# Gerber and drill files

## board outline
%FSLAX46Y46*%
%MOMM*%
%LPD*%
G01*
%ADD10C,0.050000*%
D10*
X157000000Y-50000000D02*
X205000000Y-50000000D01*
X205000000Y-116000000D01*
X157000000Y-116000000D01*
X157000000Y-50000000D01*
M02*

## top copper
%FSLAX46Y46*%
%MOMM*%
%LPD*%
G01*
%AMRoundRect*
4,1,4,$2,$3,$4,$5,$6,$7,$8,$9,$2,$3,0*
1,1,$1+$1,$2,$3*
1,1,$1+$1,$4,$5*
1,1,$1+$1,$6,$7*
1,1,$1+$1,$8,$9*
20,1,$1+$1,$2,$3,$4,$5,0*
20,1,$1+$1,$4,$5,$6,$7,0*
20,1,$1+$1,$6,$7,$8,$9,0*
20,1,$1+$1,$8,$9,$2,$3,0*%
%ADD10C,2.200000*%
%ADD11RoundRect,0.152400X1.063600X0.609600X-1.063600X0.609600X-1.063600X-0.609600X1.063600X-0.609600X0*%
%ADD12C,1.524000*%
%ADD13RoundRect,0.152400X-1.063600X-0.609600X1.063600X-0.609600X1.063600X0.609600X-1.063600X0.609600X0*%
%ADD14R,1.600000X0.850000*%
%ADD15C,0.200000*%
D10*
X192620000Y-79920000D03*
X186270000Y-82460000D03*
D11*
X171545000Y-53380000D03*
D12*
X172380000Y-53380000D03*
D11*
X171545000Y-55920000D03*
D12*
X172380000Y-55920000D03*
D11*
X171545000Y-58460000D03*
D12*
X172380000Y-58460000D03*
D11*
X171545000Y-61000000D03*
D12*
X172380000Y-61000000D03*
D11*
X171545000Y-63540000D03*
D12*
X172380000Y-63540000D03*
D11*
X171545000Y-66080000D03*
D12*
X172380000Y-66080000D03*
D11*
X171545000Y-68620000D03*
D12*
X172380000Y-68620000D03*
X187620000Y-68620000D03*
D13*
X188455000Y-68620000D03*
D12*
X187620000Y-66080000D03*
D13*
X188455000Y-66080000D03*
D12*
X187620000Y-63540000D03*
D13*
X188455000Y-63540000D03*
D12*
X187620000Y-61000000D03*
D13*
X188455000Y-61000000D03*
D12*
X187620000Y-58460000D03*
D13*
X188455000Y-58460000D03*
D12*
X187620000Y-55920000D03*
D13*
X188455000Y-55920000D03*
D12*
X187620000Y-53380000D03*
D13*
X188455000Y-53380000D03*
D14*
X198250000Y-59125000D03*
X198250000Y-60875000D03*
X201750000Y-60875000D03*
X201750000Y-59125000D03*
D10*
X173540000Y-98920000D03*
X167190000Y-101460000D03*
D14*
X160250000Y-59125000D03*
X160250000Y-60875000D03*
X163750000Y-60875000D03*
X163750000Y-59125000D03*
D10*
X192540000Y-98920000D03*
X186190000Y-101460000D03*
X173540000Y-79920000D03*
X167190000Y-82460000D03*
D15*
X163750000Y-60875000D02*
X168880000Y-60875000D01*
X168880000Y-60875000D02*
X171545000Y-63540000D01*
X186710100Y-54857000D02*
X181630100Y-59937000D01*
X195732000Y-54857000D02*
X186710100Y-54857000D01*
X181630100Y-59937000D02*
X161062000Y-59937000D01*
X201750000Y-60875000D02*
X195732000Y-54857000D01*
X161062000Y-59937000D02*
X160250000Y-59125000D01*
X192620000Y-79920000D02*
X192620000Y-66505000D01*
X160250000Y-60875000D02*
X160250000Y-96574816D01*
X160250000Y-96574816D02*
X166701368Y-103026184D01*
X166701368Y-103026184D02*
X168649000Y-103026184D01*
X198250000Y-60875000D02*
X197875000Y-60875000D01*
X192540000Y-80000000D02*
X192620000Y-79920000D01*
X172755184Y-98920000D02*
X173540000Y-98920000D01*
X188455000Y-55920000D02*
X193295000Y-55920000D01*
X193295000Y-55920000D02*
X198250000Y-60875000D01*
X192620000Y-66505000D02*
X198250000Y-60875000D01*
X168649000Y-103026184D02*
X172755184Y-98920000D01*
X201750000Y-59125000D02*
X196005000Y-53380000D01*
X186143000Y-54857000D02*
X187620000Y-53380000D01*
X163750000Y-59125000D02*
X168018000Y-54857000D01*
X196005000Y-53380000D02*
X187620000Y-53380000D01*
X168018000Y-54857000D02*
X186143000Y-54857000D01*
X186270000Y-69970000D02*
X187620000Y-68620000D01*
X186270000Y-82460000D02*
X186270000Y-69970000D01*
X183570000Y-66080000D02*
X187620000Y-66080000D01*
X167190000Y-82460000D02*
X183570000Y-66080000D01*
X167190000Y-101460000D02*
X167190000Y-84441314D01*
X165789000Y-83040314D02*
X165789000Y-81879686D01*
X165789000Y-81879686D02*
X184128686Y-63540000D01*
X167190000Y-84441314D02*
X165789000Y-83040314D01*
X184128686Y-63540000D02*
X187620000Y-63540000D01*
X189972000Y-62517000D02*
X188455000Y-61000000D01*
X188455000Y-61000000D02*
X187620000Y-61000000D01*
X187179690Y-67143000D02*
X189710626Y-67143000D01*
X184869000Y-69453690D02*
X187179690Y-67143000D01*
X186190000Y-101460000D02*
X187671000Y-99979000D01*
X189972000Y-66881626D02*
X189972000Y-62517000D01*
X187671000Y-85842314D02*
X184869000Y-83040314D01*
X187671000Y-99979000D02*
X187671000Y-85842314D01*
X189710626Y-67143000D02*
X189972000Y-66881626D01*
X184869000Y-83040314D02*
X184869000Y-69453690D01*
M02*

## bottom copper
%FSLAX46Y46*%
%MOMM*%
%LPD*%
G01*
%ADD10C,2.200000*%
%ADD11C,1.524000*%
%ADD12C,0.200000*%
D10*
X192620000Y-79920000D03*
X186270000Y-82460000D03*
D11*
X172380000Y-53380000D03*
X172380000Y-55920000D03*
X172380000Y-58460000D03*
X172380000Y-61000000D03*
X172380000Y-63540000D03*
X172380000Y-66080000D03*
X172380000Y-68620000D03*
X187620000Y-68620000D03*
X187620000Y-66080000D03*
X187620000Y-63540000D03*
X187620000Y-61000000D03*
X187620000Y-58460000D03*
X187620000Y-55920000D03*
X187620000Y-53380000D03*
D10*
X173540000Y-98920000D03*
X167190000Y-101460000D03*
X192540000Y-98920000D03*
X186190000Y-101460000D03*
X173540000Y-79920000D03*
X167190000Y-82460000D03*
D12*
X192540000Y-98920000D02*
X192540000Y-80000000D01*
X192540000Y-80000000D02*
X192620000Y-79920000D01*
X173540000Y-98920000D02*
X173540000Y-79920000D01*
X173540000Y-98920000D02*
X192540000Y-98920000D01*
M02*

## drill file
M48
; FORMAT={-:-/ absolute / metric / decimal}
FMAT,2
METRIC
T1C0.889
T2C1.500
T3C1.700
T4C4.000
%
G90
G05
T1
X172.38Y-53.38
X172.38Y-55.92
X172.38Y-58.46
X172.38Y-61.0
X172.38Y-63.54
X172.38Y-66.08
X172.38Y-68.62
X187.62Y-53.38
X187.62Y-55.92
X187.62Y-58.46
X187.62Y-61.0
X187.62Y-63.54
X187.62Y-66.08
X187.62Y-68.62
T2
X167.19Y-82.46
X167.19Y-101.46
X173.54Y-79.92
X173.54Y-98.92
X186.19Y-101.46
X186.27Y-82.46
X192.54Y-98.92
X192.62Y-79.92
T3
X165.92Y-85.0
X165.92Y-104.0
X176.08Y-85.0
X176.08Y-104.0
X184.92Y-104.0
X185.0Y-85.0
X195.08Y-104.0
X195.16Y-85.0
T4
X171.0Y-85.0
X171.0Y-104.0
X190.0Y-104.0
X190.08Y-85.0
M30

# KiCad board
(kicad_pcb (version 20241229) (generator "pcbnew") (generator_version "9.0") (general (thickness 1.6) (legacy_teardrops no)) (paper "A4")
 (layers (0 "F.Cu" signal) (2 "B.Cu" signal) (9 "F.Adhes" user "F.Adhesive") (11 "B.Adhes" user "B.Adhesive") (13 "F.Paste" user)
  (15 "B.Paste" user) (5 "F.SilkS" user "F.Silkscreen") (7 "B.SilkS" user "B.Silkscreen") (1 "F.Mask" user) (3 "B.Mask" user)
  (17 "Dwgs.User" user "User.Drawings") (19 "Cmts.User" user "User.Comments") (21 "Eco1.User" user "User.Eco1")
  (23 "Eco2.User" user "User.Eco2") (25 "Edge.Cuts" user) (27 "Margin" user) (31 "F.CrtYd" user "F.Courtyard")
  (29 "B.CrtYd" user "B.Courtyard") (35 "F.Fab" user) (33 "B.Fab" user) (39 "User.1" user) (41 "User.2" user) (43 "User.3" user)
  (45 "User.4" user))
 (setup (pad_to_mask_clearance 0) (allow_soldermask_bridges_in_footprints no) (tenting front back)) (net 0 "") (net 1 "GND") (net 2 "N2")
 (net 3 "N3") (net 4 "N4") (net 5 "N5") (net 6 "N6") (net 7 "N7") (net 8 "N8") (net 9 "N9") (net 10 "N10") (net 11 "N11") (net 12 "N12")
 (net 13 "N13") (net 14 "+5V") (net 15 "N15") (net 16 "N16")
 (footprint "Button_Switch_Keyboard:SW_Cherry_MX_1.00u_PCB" (layer "F.Cu") (at 192.62 79.92)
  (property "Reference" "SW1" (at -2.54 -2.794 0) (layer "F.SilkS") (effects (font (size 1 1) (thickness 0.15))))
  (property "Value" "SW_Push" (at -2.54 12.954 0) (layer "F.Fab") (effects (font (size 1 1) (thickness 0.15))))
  (pad "" np_thru_hole circle (at -7.62 5.08) (size 1.7 1.7) (drill 1.7) (layers "*.Cu" "*.Mask"))
  (pad "" np_thru_hole circle (at -2.54 5.08) (size 4 4) (drill 4) (layers "*.Cu" "*.Mask"))
  (pad "" np_thru_hole circle (at 2.54 5.08) (size 1.7 1.7) (drill 1.7) (layers "*.Cu" "*.Mask"))
  (pad "1" thru_hole circle (at 0 0) (size 2.2 2.2) (drill 1.5) (layers "*.Cu" "*.Mask") (remove_unused_layers no) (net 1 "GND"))
  (pad "2" thru_hole circle (at -6.35 2.54) (size 2.2 2.2) (drill 1.5) (layers "*.Cu" "*.Mask") (remove_unused_layers no) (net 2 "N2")))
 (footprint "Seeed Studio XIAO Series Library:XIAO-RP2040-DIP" (layer "F.Cu") (at 180 61)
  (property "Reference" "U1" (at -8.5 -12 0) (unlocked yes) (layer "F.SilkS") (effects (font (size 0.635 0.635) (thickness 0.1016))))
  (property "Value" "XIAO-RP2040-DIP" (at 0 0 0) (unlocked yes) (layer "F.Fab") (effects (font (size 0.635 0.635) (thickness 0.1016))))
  (pad "1" smd roundrect (at -8.455 -7.62 180) (size 2.432 1.524) (layers "F.Cu" "F.Mask") (roundrect_rratio 0.1) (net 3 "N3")
   (thermal_bridge_angle 45))
  (pad "1" thru_hole circle (at -7.62 -7.62 180) (size 1.524 1.524) (drill 0.889) (layers "*.Cu" "*.Mask") (remove_unused_layers no)
   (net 3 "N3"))
  (pad "2" smd roundrect (at -8.455 -5.08 180) (size 2.432 1.524) (layers "F.Cu" "F.Mask") (roundrect_rratio 0.1) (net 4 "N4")
   (thermal_bridge_angle 45))
  (pad "2" thru_hole circle (at -7.62 -5.08 180) (size 1.524 1.524) (drill 0.889) (layers "*.Cu" "*.Mask") (remove_unused_layers no)
   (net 4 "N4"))
  (pad "3" smd roundrect (at -8.455 -2.54 180) (size 2.432 1.524) (layers "F.Cu" "F.Mask") (roundrect_rratio 0.1) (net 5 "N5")
   (thermal_bridge_angle 45))
  (pad "3" thru_hole circle (at -7.62 -2.54 180) (size 1.524 1.524) (drill 0.889) (layers "*.Cu" "*.Mask") (remove_unused_layers no)
   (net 5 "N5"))
  (pad "4" smd roundrect (at -8.455 0 180) (size 2.432 1.524) (layers "F.Cu" "F.Mask") (roundrect_rratio 0.1) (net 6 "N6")
   (thermal_bridge_angle 45))
  (pad "4" thru_hole circle (at -7.62 0 180) (size 1.524 1.524) (drill 0.889) (layers "*.Cu" "*.Mask") (remove_unused_layers no)
   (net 6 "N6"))
  (pad "5" smd roundrect (at -8.455 2.54 180) (size 2.432 1.524) (layers "F.Cu" "F.Mask") (roundrect_rratio 0.1) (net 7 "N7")
   (thermal_bridge_angle 45))
  (pad "5" thru_hole circle (at -7.62 2.54 180) (size 1.524 1.524) (drill 0.889) (layers "*.Cu" "*.Mask") (remove_unused_layers no)
   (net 7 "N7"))
  (pad "6" smd roundrect (at -8.455 5.08 180) (size 2.432 1.524) (layers "F.Cu" "F.Mask") (roundrect_rratio 0.1) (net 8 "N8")
   (thermal_bridge_angle 45))
  (pad "6" thru_hole circle (at -7.62 5.08 180) (size 1.524 1.524) (drill 0.889) (layers "*.Cu" "*.Mask") (remove_unused_layers no)
   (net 8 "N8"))
  (pad "7" smd roundrect (at -8.455 7.62 180) (size 2.432 1.524) (layers "F.Cu" "F.Mask") (roundrect_rratio 0.1) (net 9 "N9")
   (thermal_bridge_angle 45))
  (pad "7" thru_hole circle (at -7.62 7.62 180) (size 1.524 1.524) (drill 0.889) (layers "*.Cu" "*.Mask") (remove_unused_layers no)
   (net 9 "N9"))
  (pad "8" thru_hole circle (at 7.62 7.62) (size 1.524 1.524) (drill 0.889) (layers "*.Cu" "*.Mask") (remove_unused_layers no) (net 2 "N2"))
  (pad "8" smd roundrect (at 8.455 7.62) (size 2.432 1.524) (layers "F.Cu" "F.Mask") (roundrect_rratio 0.1) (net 2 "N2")
   (thermal_bridge_angle 45))
  (pad "9" thru_hole circle (at 7.62 5.08) (size 1.524 1.524) (drill 0.889) (layers "*.Cu" "*.Mask") (remove_unused_layers no)
   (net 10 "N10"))
  (pad "9" smd roundrect (at 8.455 5.08) (size 2.432 1.524) (layers "F.Cu" "F.Mask") (roundrect_rratio 0.1) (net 10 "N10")
   (thermal_bridge_angle 45))
  (pad "10" thru_hole circle (at 7.62 2.54) (size 1.524 1.524) (drill 0.889) (layers "*.Cu" "*.Mask") (remove_unused_layers no)
   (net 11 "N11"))
  (pad "10" smd roundrect (at 8.455 2.54) (size 2.432 1.524) (layers "F.Cu" "F.Mask") (roundrect_rratio 0.1) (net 11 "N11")
   (thermal_bridge_angle 45))
  (pad "11" thru_hole circle (at 7.62 0) (size 1.524 1.524) (drill 0.889) (layers "*.Cu" "*.Mask") (remove_unused_layers no) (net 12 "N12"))
  (pad "11" smd roundrect (at 8.455 0) (size 2.432 1.524) (layers "F.Cu" "F.Mask") (roundrect_rratio 0.1) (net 12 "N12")
   (thermal_bridge_angle 45))
  (pad "12" thru_hole circle (at 7.62 -2.54) (size 1.524 1.524) (drill 0.889) (layers "*.Cu" "*.Mask") (remove_unused_layers no)
   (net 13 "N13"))
  (pad "12" smd roundrect (at 8.455 -2.54) (size 2.432 1.524) (layers "F.Cu" "F.Mask") (roundrect_rratio 0.1) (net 13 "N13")
   (thermal_bridge_angle 45))
  (pad "13" thru_hole circle (at 7.62 -5.08) (size 1.524 1.524) (drill 0.889) (layers "*.Cu" "*.Mask") (remove_unused_layers no)
   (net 1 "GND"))
  (pad "13" smd roundrect (at 8.455 -5.08) (size 2.432 1.524) (layers "F.Cu" "F.Mask") (roundrect_rratio 0.1) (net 1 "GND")
   (thermal_bridge_angle 45))
  (pad "14" thru_hole circle (at 7.62 -7.62) (size 1.524 1.524) (drill 0.889) (layers "*.Cu" "*.Mask") (remove_unused_layers no)
   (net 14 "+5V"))
  (pad "14" smd roundrect (at 8.455 -7.62) (size 2.432 1.524) (layers "F.Cu" "F.Mask") (roundrect_rratio 0.1) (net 14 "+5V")
   (thermal_bridge_angle 45)))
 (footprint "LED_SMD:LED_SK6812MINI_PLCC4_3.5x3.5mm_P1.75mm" (layer "F.Cu") (at 200 60)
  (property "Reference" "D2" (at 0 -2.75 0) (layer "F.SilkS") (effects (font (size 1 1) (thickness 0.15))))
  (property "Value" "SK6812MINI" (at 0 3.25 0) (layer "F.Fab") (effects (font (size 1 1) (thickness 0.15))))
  (pad "1" smd rect (at -1.75 -0.875) (size 1.6 0.85) (layers "F.Cu" "F.Mask" "F.Paste") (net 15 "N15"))
  (pad "2" smd rect (at -1.75 0.875) (size 1.6 0.85) (layers "F.Cu" "F.Mask" "F.Paste") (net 1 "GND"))
  (pad "3" smd rect (at 1.75 0.875) (size 1.6 0.85) (layers "F.Cu" "F.Mask" "F.Paste") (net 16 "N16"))
  (pad "4" smd rect (at 1.75 -0.875) (size 1.6 0.85) (layers "F.Cu" "F.Mask" "F.Paste") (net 14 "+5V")))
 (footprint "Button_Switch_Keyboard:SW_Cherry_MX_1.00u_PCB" (layer "F.Cu") (at 173.54 98.92)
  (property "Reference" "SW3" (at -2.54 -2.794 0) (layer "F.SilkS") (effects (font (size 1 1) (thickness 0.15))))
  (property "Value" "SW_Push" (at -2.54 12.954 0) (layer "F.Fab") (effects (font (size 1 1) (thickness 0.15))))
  (pad "" np_thru_hole circle (at -7.62 5.08) (size 1.7 1.7) (drill 1.7) (layers "*.Cu" "*.Mask"))
  (pad "" np_thru_hole circle (at -2.54 5.08) (size 4 4) (drill 4) (layers "*.Cu" "*.Mask"))
  (pad "" np_thru_hole circle (at 2.54 5.08) (size 1.7 1.7) (drill 1.7) (layers "*.Cu" "*.Mask"))
  (pad "1" thru_hole circle (at 0 0) (size 2.2 2.2) (drill 1.5) (layers "*.Cu" "*.Mask") (remove_unused_layers no) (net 1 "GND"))
  (pad "2" thru_hole circle (at -6.35 2.54) (size 2.2 2.2) (drill 1.5) (layers "*.Cu" "*.Mask") (remove_unused_layers no) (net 11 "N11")))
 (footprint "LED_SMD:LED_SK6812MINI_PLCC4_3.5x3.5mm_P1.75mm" (layer "F.Cu") (at 162 60)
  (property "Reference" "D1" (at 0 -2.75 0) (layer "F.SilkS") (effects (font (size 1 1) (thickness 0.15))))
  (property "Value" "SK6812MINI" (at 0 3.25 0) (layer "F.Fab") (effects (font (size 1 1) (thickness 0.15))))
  (pad "1" smd rect (at -1.75 -0.875) (size 1.6 0.85) (layers "F.Cu" "F.Mask" "F.Paste") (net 16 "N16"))
  (pad "2" smd rect (at -1.75 0.875) (size 1.6 0.85) (layers "F.Cu" "F.Mask" "F.Paste") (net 1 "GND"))
  (pad "3" smd rect (at 1.75 0.875) (size 1.6 0.85) (layers "F.Cu" "F.Mask" "F.Paste") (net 7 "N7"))
  (pad "4" smd rect (at 1.75 -0.875) (size 1.6 0.85) (layers "F.Cu" "F.Mask" "F.Paste") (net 14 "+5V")))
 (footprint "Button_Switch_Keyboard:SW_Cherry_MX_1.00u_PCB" (layer "F.Cu") (at 192.54 98.92)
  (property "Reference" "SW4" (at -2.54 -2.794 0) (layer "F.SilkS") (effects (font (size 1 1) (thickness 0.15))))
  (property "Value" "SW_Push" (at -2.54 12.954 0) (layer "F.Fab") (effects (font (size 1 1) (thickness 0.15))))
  (pad "" np_thru_hole circle (at -7.62 5.08) (size 1.7 1.7) (drill 1.7) (layers "*.Cu" "*.Mask"))
  (pad "" np_thru_hole circle (at -2.54 5.08) (size 4 4) (drill 4) (layers "*.Cu" "*.Mask"))
  (pad "" np_thru_hole circle (at 2.54 5.08) (size 1.7 1.7) (drill 1.7) (layers "*.Cu" "*.Mask"))
  (pad "1" thru_hole circle (at 0 0) (size 2.2 2.2) (drill 1.5) (layers "*.Cu" "*.Mask") (remove_unused_layers no) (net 1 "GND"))
  (pad "2" thru_hole circle (at -6.35 2.54) (size 2.2 2.2) (drill 1.5) (layers "*.Cu" "*.Mask") (remove_unused_layers no) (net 12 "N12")))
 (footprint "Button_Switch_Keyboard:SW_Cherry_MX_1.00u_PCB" (layer "F.Cu") (at 173.54 79.92)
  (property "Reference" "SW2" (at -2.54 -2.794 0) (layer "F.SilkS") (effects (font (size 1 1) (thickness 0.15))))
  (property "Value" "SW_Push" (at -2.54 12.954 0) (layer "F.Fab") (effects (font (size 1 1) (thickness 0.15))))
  (pad "" np_thru_hole circle (at -7.62 5.08) (size 1.7 1.7) (drill 1.7) (layers "*.Cu" "*.Mask"))
  (pad "" np_thru_hole circle (at -2.54 5.08) (size 4 4) (drill 4) (layers "*.Cu" "*.Mask"))
  (pad "" np_thru_hole circle (at 2.54 5.08) (size 1.7 1.7) (drill 1.7) (layers "*.Cu" "*.Mask"))
  (pad "1" thru_hole circle (at 0 0) (size 2.2 2.2) (drill 1.5) (layers "*.Cu" "*.Mask") (remove_unused_layers no) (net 1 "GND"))
  (pad "2" thru_hole circle (at -6.35 2.54) (size 2.2 2.2) (drill 1.5) (layers "*.Cu" "*.Mask") (remove_unused_layers no) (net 10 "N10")))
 (gr_rect (start 157 50) (end 205 116) (stroke (width 0.05) (type default)) (fill no) (layer "Edge.Cuts"))
 (segment (start 163.75 60.875) (end 168.88 60.875) (width 0.2) (layer "F.Cu") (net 7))
 (segment (start 168.88 60.875) (end 171.545 63.54) (width 0.2) (layer "F.Cu") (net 7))
 (segment (start 186.7101 54.857) (end 181.6301 59.937) (width 0.2) (layer "F.Cu") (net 16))
 (segment (start 195.732 54.857) (end 186.7101 54.857) (width 0.2) (layer "F.Cu") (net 16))
 (segment (start 181.6301 59.937) (end 161.062 59.937) (width 0.2) (layer "F.Cu") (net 16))
 (segment (start 201.75 60.875) (end 195.732 54.857) (width 0.2) (layer "F.Cu") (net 16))
 (segment (start 161.062 59.937) (end 160.25 59.125) (width 0.2) (layer "F.Cu") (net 16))
 (segment (start 192.62 79.92) (end 192.62 66.505) (width 0.2) (layer "F.Cu") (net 1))
 (segment (start 160.25 60.875) (end 160.25 96.574816) (width 0.2) (layer "F.Cu") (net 1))
 (segment (start 160.25 96.574816) (end 166.701368 103.026184) (width 0.2) (layer "F.Cu") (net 1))
 (segment (start 166.701368 103.026184) (end 168.649 103.026184) (width 0.2) (layer "F.Cu") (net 1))
 (segment (start 198.25 60.875) (end 197.875 60.875) (width 0.2) (layer "F.Cu") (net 1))
 (segment (start 192.54 80) (end 192.62 79.92) (width 0.2) (layer "F.Cu") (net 1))
 (segment (start 172.755184 98.92) (end 173.54 98.92) (width 0.2) (layer "F.Cu") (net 1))
 (segment (start 188.455 55.92) (end 193.295 55.92) (width 0.2) (layer "F.Cu") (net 1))
 (segment (start 193.295 55.92) (end 198.25 60.875) (width 0.2) (layer "F.Cu") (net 1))
 (segment (start 192.62 66.505) (end 198.25 60.875) (width 0.2) (layer "F.Cu") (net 1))
 (segment (start 168.649 103.026184) (end 172.755184 98.92) (width 0.2) (layer "F.Cu") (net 1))
 (segment (start 192.54 98.92) (end 192.54 80) (width 0.2) (layer "B.Cu") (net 1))
 (segment (start 192.54 80) (end 192.62 79.92) (width 0.2) (layer "B.Cu") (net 1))
 (segment (start 173.54 98.92) (end 173.54 79.92) (width 0.2) (layer "B.Cu") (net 1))
 (segment (start 173.54 98.92) (end 192.54 98.92) (width 0.2) (layer "B.Cu") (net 1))
 (segment (start 201.75 59.125) (end 196.005 53.38) (width 0.2) (layer "F.Cu") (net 14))
 (segment (start 186.143 54.857) (end 187.62 53.38) (width 0.2) (layer "F.Cu") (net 14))
 (segment (start 163.75 59.125) (end 168.018 54.857) (width 0.2) (layer "F.Cu") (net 14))
 (segment (start 196.005 53.38) (end 187.62 53.38) (width 0.2) (layer "F.Cu") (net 14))
 (segment (start 168.018 54.857) (end 186.143 54.857) (width 0.2) (layer "F.Cu") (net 14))
 (segment (start 186.27 69.97) (end 187.62 68.62) (width 0.2) (layer "F.Cu") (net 2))
 (segment (start 186.27 82.46) (end 186.27 69.97) (width 0.2) (layer "F.Cu") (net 2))
 (segment (start 183.57 66.08) (end 187.62 66.08) (width 0.2) (layer "F.Cu") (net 10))
 (segment (start 167.19 82.46) (end 183.57 66.08) (width 0.2) (layer "F.Cu") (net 10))
 (segment (start 167.19 101.46) (end 167.19 84.441314) (width 0.2) (layer "F.Cu") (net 11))
 (segment (start 165.789 83.040314) (end 165.789 81.879686) (width 0.2) (layer "F.Cu") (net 11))
 (segment (start 165.789 81.879686) (end 184.128686 63.54) (width 0.2) (layer "F.Cu") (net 11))
 (segment (start 167.19 84.441314) (end 165.789 83.040314) (width 0.2) (layer "F.Cu") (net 11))
 (segment (start 184.128686 63.54) (end 187.62 63.54) (width 0.2) (layer "F.Cu") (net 11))
 (segment (start 189.972 62.517) (end 188.455 61) (width 0.2) (layer "F.Cu") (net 12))
 (segment (start 188.455 61) (end 187.62 61) (width 0.2) (layer "F.Cu") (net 12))
 (segment (start 187.17969 67.143) (end 189.710626 67.143) (width 0.2) (layer "F.Cu") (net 12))
 (segment (start 184.869 69.45369) (end 187.17969 67.143) (width 0.2) (layer "F.Cu") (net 12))
 (segment (start 186.19 101.46) (end 187.671 99.979) (width 0.2) (layer "F.Cu") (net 12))
 (segment (start 189.972 66.881626) (end 189.972 62.517) (width 0.2) (layer "F.Cu") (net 12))
 (segment (start 187.671 85.842314) (end 184.869 83.040314) (width 0.2) (layer "F.Cu") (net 12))
 (segment (start 187.671 99.979) (end 187.671 85.842314) (width 0.2) (layer "F.Cu") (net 12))
 (segment (start 189.710626 67.143) (end 189.972 66.881626) (width 0.2) (layer "F.Cu") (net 12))
 (segment (start 184.869 83.040314) (end 184.869 69.45369) (width 0.2) (layer "F.Cu") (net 12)))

